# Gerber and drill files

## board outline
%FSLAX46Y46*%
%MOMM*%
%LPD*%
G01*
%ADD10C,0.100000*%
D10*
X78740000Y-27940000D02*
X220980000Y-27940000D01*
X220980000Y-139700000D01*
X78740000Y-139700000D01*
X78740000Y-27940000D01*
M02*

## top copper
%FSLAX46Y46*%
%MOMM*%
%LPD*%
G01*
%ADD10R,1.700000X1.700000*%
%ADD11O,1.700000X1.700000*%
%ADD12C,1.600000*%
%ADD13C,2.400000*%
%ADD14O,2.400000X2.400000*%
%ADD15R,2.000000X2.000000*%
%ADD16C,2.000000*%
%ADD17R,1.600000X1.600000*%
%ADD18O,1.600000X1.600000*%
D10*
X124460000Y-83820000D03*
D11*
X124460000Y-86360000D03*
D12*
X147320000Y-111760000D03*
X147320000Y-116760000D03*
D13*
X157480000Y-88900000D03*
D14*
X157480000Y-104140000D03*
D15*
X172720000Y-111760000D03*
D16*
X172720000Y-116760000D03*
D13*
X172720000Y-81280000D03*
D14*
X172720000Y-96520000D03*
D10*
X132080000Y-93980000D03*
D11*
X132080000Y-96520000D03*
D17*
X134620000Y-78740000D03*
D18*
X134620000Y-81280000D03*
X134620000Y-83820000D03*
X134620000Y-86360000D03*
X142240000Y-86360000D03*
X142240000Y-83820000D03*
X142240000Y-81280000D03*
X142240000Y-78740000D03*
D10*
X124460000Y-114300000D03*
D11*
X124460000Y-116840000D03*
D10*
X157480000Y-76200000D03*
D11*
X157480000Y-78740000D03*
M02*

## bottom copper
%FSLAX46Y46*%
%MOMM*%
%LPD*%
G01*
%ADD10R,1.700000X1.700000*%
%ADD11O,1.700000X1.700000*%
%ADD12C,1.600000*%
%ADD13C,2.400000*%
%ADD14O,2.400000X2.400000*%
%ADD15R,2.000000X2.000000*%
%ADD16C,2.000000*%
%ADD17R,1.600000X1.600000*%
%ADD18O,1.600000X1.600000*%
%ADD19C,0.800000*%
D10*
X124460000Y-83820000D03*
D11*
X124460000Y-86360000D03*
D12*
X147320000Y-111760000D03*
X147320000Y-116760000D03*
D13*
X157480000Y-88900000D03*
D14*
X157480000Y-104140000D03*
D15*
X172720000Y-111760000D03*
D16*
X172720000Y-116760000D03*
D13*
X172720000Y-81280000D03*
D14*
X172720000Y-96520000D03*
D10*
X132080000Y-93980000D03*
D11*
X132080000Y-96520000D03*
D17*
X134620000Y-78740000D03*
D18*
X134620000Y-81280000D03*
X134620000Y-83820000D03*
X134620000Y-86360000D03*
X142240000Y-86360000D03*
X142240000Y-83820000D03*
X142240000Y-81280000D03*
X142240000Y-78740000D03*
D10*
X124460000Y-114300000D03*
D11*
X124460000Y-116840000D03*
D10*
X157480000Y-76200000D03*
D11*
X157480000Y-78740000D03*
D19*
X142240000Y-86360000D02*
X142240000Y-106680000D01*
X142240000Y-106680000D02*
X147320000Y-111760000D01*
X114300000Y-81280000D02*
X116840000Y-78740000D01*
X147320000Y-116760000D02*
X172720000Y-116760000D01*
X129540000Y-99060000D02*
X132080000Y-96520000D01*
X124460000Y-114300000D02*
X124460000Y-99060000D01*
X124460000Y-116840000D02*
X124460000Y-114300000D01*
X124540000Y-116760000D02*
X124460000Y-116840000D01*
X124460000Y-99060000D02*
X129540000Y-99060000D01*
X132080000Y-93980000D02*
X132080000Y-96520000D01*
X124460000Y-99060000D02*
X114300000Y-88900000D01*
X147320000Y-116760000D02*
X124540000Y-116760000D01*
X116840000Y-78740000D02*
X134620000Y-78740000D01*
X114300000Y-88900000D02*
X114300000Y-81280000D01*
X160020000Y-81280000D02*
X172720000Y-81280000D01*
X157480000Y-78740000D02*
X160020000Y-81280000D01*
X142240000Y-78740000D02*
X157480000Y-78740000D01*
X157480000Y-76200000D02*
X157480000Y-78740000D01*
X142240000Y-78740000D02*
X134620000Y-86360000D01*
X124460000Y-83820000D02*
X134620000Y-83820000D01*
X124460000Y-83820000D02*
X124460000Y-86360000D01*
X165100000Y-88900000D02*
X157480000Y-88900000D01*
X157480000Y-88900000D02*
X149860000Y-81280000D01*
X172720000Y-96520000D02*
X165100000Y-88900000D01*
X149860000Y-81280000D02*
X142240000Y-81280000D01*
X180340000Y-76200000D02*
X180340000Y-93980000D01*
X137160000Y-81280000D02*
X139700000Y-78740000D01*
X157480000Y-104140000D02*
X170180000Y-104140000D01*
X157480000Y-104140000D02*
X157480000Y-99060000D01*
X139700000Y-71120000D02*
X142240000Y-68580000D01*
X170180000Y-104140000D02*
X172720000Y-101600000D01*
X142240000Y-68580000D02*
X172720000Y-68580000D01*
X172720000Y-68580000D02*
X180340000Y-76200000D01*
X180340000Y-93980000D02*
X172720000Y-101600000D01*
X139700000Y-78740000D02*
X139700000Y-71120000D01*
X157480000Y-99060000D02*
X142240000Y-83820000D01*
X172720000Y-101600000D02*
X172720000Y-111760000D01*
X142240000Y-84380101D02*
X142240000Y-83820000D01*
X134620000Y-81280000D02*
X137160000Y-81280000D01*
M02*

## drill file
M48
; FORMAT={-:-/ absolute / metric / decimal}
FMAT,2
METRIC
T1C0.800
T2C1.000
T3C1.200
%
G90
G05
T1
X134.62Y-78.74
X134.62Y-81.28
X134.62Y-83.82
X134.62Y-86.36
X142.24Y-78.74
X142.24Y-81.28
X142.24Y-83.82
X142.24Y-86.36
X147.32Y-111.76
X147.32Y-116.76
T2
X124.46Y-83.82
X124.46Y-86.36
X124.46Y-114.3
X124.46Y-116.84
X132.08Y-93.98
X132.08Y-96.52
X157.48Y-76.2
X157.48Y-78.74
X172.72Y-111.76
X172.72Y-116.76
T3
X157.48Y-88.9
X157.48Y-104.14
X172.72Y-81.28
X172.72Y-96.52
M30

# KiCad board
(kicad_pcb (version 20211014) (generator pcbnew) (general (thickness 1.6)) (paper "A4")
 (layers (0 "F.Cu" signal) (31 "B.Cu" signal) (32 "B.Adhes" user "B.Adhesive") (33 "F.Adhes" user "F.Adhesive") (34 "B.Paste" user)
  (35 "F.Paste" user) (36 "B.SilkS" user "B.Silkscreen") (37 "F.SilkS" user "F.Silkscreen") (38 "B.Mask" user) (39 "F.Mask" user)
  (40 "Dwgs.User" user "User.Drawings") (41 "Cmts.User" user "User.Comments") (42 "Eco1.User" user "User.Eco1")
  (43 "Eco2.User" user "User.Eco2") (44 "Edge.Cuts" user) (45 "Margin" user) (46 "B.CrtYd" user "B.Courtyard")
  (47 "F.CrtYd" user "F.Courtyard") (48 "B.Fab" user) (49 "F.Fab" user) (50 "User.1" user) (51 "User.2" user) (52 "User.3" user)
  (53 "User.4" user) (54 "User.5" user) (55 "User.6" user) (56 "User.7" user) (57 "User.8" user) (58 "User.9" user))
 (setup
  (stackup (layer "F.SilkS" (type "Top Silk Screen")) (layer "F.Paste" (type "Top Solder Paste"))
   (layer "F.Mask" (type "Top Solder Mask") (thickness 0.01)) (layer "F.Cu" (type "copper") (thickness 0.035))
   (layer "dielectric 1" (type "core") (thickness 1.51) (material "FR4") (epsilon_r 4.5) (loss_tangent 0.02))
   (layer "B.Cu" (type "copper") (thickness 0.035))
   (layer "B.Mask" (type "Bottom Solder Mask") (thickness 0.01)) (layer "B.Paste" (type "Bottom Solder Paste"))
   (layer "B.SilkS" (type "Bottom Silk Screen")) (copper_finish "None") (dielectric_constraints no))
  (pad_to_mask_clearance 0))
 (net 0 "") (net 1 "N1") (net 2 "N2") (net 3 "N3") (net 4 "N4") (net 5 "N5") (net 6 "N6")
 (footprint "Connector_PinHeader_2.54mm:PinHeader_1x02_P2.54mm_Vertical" (layer "F.Cu") (at 124.46 83.82)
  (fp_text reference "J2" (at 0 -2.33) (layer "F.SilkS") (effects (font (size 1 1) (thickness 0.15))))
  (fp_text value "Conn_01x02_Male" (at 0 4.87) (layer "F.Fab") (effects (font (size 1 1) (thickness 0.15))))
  (pad "1" thru_hole rect (at 0 0) (size 1.7 1.7) (drill 1) (layers *.Cu *.Mask) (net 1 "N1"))
  (pad "2" thru_hole oval (at 0 2.54) (size 1.7 1.7) (drill 1) (layers *.Cu *.Mask) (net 1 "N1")))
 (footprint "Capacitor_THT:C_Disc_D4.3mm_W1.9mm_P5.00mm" (layer "F.Cu") (at 147.32 111.76 -90)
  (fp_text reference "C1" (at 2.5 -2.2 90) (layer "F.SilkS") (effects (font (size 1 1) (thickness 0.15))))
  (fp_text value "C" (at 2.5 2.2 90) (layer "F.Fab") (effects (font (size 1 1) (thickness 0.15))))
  (pad "1" thru_hole circle (at 0 0 270) (size 1.6 1.6) (drill 0.8) (layers *.Cu *.Mask) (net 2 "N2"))
  (pad "2" thru_hole circle (at 5 0 270) (size 1.6 1.6) (drill 0.8) (layers *.Cu *.Mask) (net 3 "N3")))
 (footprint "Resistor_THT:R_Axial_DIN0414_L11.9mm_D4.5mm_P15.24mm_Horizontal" (layer "F.Cu") (at 157.48 88.9 -90)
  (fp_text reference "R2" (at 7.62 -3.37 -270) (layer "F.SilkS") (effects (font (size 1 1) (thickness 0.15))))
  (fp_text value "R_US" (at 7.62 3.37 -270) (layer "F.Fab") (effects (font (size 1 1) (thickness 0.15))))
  (pad "1" thru_hole circle (at 0 0 270) (size 2.4 2.4) (drill 1.2) (layers *.Cu *.Mask) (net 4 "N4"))
  (pad "2" thru_hole oval (at 15.24 0 270) (size 2.4 2.4) (drill 1.2) (layers *.Cu *.Mask) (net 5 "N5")))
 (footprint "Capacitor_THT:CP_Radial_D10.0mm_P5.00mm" (layer "F.Cu") (at 172.72 111.76 -90)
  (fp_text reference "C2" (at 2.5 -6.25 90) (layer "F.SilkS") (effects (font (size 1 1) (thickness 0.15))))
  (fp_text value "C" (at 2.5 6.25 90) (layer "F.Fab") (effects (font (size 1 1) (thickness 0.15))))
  (pad "1" thru_hole rect (at 0 0 270) (size 2 2) (drill 1) (layers *.Cu *.Mask) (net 5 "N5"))
  (pad "2" thru_hole circle (at 5 0 270) (size 2 2) (drill 1) (layers *.Cu *.Mask) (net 3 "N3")))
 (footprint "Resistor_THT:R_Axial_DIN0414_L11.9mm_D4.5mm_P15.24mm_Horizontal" (layer "F.Cu") (at 172.72 81.28 -90)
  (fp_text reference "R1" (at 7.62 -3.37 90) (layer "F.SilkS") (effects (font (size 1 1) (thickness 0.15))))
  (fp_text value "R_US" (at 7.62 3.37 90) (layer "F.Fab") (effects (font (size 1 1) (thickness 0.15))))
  (pad "1" thru_hole circle (at 0 0 270) (size 2.4 2.4) (drill 1.2) (layers *.Cu *.Mask) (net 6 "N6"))
  (pad "2" thru_hole oval (at 15.24 0 270) (size 2.4 2.4) (drill 1.2) (layers *.Cu *.Mask) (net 4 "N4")))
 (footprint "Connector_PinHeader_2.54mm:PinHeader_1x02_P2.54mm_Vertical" (layer "F.Cu") (at 132.08 93.98)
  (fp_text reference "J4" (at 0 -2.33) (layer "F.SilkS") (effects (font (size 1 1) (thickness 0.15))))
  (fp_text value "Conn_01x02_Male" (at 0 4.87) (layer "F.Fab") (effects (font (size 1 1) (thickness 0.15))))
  (pad "1" thru_hole rect (at 0 0) (size 1.7 1.7) (drill 1) (layers *.Cu *.Mask) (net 3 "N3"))
  (pad "2" thru_hole oval (at 0 2.54) (size 1.7 1.7) (drill 1) (layers *.Cu *.Mask) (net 3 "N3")))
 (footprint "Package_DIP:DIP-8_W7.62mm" (layer "F.Cu") (at 134.62 78.74)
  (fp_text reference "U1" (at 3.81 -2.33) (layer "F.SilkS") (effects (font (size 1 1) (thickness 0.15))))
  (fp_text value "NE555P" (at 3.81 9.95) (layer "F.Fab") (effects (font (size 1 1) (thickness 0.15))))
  (pad "1" thru_hole rect (at 0 0) (size 1.6 1.6) (drill 0.8) (layers *.Cu *.Mask) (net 3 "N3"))
  (pad "2" thru_hole oval (at 0 2.54) (size 1.6 1.6) (drill 0.8) (layers *.Cu *.Mask) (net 5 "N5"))
  (pad "3" thru_hole oval (at 0 5.08) (size 1.6 1.6) (drill 0.8) (layers *.Cu *.Mask) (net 1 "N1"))
  (pad "4" thru_hole oval (at 0 7.62) (size 1.6 1.6) (drill 0.8) (layers *.Cu *.Mask) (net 6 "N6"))
  (pad "5" thru_hole oval (at 7.62 7.62) (size 1.6 1.6) (drill 0.8) (layers *.Cu *.Mask) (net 2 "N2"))
  (pad "6" thru_hole oval (at 7.62 5.08) (size 1.6 1.6) (drill 0.8) (layers *.Cu *.Mask) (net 5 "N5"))
  (pad "7" thru_hole oval (at 7.62 2.54) (size 1.6 1.6) (drill 0.8) (layers *.Cu *.Mask) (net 4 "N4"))
  (pad "8" thru_hole oval (at 7.62 0) (size 1.6 1.6) (drill 0.8) (layers *.Cu *.Mask) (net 6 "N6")))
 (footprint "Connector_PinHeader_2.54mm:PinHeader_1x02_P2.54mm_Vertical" (layer "F.Cu") (at 124.46 114.3)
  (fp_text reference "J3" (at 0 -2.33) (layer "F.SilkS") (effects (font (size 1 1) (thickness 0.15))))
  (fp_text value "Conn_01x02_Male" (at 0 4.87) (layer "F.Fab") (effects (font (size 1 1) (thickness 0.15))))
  (pad "1" thru_hole rect (at 0 0) (size 1.7 1.7) (drill 1) (layers *.Cu *.Mask) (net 3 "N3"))
  (pad "2" thru_hole oval (at 0 2.54) (size 1.7 1.7) (drill 1) (layers *.Cu *.Mask) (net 3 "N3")))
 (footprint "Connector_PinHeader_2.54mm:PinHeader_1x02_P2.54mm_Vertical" (layer "F.Cu") (at 157.48 76.2)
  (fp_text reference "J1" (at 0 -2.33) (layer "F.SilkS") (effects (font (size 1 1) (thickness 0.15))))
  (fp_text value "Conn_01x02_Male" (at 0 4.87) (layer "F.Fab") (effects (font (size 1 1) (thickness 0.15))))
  (pad "1" thru_hole rect (at 0 0) (size 1.7 1.7) (drill 1) (layers *.Cu *.Mask) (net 6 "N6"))
  (pad "2" thru_hole oval (at 0 2.54) (size 1.7 1.7) (drill 1) (layers *.Cu *.Mask) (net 6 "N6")))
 (gr_rect (start 78.74 27.94) (end 220.98 139.7) (layer "Edge.Cuts") (width 0.1) (fill none))
 (segment (start 142.24 86.36) (end 142.24 106.68) (width 0.8) (layer "B.Cu") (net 2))
 (segment (start 142.24 106.68) (end 147.32 111.76) (width 0.8) (layer "B.Cu") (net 2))
 (segment (start 114.3 81.28) (end 116.84 78.74) (width 0.8) (layer "B.Cu") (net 3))
 (segment (start 147.32 116.76) (end 172.72 116.76) (width 0.8) (layer "B.Cu") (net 3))
 (segment (start 129.54 99.06) (end 132.08 96.52) (width 0.8) (layer "B.Cu") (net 3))
 (segment (start 124.46 114.3) (end 124.46 99.06) (width 0.8) (layer "B.Cu") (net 3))
 (segment (start 124.46 116.84) (end 124.46 114.3) (width 0.8) (layer "B.Cu") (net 3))
 (segment (start 124.54 116.76) (end 124.46 116.84) (width 0.8) (layer "B.Cu") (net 3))
 (segment (start 124.46 99.06) (end 129.54 99.06) (width 0.8) (layer "B.Cu") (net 3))
 (segment (start 132.08 93.98) (end 132.08 96.52) (width 0.8) (layer "B.Cu") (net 3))
 (segment (start 124.46 99.06) (end 114.3 88.9) (width 0.8) (layer "B.Cu") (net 3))
 (segment (start 147.32 116.76) (end 124.54 116.76) (width 0.8) (layer "B.Cu") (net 3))
 (segment (start 116.84 78.74) (end 134.62 78.74) (width 0.8) (layer "B.Cu") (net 3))
 (segment (start 114.3 88.9) (end 114.3 81.28) (width 0.8) (layer "B.Cu") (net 3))
 (segment (start 160.02 81.28) (end 172.72 81.28) (width 0.8) (layer "B.Cu") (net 6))
 (segment (start 157.48 78.74) (end 160.02 81.28) (width 0.8) (layer "B.Cu") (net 6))
 (segment (start 142.24 78.74) (end 157.48 78.74) (width 0.8) (layer "B.Cu") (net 6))
 (segment (start 157.48 76.2) (end 157.48 78.74) (width 0.8) (layer "B.Cu") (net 6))
 (segment (start 142.24 78.74) (end 134.62 86.36) (width 0.8) (layer "B.Cu") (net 6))
 (segment (start 124.46 83.82) (end 134.62 83.82) (width 0.8) (layer "B.Cu") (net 1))
 (segment (start 124.46 83.82) (end 124.46 86.36) (width 0.8) (layer "B.Cu") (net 1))
 (segment (start 165.1 88.9) (end 157.48 88.9) (width 0.8) (layer "B.Cu") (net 4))
 (segment (start 157.48 88.9) (end 149.86 81.28) (width 0.8) (layer "B.Cu") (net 4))
 (segment (start 172.72 96.52) (end 165.1 88.9) (width 0.8) (layer "B.Cu") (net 4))
 (segment (start 149.86 81.28) (end 142.24 81.28) (width 0.8) (layer "B.Cu") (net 4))
 (segment (start 180.34 76.2) (end 180.34 93.98) (width 0.8) (layer "B.Cu") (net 5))
 (segment (start 137.16 81.28) (end 139.7 78.74) (width 0.8) (layer "B.Cu") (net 5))
 (segment (start 157.48 104.14) (end 170.18 104.14) (width 0.8) (layer "B.Cu") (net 5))
 (segment (start 157.48 104.14) (end 157.48 99.06) (width 0.8) (layer "B.Cu") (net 5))
 (segment (start 139.7 71.12) (end 142.24 68.58) (width 0.8) (layer "B.Cu") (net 5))
 (segment (start 170.18 104.14) (end 172.72 101.6) (width 0.8) (layer "B.Cu") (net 5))
 (segment (start 142.24 68.58) (end 172.72 68.58) (width 0.8) (layer "B.Cu") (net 5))
 (segment (start 172.72 68.58) (end 180.34 76.2) (width 0.8) (layer "B.Cu") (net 5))
 (segment (start 180.34 93.98) (end 172.72 101.6) (width 0.8) (layer "B.Cu") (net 5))
 (segment (start 139.7 78.74) (end 139.7 71.12) (width 0.8) (layer "B.Cu") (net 5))
 (segment (start 157.48 99.06) (end 142.24 83.82) (width 0.8) (layer "B.Cu") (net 5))
 (segment (start 172.72 101.6) (end 172.72 111.76) (width 0.8) (layer "B.Cu") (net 5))
 (segment (start 142.24 84.380101) (end 142.24 83.82) (width 0.8) (layer "B.Cu") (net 5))
 (segment (start 134.62 81.28) (end 137.16 81.28) (width 0.8) (layer "B.Cu") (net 5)))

